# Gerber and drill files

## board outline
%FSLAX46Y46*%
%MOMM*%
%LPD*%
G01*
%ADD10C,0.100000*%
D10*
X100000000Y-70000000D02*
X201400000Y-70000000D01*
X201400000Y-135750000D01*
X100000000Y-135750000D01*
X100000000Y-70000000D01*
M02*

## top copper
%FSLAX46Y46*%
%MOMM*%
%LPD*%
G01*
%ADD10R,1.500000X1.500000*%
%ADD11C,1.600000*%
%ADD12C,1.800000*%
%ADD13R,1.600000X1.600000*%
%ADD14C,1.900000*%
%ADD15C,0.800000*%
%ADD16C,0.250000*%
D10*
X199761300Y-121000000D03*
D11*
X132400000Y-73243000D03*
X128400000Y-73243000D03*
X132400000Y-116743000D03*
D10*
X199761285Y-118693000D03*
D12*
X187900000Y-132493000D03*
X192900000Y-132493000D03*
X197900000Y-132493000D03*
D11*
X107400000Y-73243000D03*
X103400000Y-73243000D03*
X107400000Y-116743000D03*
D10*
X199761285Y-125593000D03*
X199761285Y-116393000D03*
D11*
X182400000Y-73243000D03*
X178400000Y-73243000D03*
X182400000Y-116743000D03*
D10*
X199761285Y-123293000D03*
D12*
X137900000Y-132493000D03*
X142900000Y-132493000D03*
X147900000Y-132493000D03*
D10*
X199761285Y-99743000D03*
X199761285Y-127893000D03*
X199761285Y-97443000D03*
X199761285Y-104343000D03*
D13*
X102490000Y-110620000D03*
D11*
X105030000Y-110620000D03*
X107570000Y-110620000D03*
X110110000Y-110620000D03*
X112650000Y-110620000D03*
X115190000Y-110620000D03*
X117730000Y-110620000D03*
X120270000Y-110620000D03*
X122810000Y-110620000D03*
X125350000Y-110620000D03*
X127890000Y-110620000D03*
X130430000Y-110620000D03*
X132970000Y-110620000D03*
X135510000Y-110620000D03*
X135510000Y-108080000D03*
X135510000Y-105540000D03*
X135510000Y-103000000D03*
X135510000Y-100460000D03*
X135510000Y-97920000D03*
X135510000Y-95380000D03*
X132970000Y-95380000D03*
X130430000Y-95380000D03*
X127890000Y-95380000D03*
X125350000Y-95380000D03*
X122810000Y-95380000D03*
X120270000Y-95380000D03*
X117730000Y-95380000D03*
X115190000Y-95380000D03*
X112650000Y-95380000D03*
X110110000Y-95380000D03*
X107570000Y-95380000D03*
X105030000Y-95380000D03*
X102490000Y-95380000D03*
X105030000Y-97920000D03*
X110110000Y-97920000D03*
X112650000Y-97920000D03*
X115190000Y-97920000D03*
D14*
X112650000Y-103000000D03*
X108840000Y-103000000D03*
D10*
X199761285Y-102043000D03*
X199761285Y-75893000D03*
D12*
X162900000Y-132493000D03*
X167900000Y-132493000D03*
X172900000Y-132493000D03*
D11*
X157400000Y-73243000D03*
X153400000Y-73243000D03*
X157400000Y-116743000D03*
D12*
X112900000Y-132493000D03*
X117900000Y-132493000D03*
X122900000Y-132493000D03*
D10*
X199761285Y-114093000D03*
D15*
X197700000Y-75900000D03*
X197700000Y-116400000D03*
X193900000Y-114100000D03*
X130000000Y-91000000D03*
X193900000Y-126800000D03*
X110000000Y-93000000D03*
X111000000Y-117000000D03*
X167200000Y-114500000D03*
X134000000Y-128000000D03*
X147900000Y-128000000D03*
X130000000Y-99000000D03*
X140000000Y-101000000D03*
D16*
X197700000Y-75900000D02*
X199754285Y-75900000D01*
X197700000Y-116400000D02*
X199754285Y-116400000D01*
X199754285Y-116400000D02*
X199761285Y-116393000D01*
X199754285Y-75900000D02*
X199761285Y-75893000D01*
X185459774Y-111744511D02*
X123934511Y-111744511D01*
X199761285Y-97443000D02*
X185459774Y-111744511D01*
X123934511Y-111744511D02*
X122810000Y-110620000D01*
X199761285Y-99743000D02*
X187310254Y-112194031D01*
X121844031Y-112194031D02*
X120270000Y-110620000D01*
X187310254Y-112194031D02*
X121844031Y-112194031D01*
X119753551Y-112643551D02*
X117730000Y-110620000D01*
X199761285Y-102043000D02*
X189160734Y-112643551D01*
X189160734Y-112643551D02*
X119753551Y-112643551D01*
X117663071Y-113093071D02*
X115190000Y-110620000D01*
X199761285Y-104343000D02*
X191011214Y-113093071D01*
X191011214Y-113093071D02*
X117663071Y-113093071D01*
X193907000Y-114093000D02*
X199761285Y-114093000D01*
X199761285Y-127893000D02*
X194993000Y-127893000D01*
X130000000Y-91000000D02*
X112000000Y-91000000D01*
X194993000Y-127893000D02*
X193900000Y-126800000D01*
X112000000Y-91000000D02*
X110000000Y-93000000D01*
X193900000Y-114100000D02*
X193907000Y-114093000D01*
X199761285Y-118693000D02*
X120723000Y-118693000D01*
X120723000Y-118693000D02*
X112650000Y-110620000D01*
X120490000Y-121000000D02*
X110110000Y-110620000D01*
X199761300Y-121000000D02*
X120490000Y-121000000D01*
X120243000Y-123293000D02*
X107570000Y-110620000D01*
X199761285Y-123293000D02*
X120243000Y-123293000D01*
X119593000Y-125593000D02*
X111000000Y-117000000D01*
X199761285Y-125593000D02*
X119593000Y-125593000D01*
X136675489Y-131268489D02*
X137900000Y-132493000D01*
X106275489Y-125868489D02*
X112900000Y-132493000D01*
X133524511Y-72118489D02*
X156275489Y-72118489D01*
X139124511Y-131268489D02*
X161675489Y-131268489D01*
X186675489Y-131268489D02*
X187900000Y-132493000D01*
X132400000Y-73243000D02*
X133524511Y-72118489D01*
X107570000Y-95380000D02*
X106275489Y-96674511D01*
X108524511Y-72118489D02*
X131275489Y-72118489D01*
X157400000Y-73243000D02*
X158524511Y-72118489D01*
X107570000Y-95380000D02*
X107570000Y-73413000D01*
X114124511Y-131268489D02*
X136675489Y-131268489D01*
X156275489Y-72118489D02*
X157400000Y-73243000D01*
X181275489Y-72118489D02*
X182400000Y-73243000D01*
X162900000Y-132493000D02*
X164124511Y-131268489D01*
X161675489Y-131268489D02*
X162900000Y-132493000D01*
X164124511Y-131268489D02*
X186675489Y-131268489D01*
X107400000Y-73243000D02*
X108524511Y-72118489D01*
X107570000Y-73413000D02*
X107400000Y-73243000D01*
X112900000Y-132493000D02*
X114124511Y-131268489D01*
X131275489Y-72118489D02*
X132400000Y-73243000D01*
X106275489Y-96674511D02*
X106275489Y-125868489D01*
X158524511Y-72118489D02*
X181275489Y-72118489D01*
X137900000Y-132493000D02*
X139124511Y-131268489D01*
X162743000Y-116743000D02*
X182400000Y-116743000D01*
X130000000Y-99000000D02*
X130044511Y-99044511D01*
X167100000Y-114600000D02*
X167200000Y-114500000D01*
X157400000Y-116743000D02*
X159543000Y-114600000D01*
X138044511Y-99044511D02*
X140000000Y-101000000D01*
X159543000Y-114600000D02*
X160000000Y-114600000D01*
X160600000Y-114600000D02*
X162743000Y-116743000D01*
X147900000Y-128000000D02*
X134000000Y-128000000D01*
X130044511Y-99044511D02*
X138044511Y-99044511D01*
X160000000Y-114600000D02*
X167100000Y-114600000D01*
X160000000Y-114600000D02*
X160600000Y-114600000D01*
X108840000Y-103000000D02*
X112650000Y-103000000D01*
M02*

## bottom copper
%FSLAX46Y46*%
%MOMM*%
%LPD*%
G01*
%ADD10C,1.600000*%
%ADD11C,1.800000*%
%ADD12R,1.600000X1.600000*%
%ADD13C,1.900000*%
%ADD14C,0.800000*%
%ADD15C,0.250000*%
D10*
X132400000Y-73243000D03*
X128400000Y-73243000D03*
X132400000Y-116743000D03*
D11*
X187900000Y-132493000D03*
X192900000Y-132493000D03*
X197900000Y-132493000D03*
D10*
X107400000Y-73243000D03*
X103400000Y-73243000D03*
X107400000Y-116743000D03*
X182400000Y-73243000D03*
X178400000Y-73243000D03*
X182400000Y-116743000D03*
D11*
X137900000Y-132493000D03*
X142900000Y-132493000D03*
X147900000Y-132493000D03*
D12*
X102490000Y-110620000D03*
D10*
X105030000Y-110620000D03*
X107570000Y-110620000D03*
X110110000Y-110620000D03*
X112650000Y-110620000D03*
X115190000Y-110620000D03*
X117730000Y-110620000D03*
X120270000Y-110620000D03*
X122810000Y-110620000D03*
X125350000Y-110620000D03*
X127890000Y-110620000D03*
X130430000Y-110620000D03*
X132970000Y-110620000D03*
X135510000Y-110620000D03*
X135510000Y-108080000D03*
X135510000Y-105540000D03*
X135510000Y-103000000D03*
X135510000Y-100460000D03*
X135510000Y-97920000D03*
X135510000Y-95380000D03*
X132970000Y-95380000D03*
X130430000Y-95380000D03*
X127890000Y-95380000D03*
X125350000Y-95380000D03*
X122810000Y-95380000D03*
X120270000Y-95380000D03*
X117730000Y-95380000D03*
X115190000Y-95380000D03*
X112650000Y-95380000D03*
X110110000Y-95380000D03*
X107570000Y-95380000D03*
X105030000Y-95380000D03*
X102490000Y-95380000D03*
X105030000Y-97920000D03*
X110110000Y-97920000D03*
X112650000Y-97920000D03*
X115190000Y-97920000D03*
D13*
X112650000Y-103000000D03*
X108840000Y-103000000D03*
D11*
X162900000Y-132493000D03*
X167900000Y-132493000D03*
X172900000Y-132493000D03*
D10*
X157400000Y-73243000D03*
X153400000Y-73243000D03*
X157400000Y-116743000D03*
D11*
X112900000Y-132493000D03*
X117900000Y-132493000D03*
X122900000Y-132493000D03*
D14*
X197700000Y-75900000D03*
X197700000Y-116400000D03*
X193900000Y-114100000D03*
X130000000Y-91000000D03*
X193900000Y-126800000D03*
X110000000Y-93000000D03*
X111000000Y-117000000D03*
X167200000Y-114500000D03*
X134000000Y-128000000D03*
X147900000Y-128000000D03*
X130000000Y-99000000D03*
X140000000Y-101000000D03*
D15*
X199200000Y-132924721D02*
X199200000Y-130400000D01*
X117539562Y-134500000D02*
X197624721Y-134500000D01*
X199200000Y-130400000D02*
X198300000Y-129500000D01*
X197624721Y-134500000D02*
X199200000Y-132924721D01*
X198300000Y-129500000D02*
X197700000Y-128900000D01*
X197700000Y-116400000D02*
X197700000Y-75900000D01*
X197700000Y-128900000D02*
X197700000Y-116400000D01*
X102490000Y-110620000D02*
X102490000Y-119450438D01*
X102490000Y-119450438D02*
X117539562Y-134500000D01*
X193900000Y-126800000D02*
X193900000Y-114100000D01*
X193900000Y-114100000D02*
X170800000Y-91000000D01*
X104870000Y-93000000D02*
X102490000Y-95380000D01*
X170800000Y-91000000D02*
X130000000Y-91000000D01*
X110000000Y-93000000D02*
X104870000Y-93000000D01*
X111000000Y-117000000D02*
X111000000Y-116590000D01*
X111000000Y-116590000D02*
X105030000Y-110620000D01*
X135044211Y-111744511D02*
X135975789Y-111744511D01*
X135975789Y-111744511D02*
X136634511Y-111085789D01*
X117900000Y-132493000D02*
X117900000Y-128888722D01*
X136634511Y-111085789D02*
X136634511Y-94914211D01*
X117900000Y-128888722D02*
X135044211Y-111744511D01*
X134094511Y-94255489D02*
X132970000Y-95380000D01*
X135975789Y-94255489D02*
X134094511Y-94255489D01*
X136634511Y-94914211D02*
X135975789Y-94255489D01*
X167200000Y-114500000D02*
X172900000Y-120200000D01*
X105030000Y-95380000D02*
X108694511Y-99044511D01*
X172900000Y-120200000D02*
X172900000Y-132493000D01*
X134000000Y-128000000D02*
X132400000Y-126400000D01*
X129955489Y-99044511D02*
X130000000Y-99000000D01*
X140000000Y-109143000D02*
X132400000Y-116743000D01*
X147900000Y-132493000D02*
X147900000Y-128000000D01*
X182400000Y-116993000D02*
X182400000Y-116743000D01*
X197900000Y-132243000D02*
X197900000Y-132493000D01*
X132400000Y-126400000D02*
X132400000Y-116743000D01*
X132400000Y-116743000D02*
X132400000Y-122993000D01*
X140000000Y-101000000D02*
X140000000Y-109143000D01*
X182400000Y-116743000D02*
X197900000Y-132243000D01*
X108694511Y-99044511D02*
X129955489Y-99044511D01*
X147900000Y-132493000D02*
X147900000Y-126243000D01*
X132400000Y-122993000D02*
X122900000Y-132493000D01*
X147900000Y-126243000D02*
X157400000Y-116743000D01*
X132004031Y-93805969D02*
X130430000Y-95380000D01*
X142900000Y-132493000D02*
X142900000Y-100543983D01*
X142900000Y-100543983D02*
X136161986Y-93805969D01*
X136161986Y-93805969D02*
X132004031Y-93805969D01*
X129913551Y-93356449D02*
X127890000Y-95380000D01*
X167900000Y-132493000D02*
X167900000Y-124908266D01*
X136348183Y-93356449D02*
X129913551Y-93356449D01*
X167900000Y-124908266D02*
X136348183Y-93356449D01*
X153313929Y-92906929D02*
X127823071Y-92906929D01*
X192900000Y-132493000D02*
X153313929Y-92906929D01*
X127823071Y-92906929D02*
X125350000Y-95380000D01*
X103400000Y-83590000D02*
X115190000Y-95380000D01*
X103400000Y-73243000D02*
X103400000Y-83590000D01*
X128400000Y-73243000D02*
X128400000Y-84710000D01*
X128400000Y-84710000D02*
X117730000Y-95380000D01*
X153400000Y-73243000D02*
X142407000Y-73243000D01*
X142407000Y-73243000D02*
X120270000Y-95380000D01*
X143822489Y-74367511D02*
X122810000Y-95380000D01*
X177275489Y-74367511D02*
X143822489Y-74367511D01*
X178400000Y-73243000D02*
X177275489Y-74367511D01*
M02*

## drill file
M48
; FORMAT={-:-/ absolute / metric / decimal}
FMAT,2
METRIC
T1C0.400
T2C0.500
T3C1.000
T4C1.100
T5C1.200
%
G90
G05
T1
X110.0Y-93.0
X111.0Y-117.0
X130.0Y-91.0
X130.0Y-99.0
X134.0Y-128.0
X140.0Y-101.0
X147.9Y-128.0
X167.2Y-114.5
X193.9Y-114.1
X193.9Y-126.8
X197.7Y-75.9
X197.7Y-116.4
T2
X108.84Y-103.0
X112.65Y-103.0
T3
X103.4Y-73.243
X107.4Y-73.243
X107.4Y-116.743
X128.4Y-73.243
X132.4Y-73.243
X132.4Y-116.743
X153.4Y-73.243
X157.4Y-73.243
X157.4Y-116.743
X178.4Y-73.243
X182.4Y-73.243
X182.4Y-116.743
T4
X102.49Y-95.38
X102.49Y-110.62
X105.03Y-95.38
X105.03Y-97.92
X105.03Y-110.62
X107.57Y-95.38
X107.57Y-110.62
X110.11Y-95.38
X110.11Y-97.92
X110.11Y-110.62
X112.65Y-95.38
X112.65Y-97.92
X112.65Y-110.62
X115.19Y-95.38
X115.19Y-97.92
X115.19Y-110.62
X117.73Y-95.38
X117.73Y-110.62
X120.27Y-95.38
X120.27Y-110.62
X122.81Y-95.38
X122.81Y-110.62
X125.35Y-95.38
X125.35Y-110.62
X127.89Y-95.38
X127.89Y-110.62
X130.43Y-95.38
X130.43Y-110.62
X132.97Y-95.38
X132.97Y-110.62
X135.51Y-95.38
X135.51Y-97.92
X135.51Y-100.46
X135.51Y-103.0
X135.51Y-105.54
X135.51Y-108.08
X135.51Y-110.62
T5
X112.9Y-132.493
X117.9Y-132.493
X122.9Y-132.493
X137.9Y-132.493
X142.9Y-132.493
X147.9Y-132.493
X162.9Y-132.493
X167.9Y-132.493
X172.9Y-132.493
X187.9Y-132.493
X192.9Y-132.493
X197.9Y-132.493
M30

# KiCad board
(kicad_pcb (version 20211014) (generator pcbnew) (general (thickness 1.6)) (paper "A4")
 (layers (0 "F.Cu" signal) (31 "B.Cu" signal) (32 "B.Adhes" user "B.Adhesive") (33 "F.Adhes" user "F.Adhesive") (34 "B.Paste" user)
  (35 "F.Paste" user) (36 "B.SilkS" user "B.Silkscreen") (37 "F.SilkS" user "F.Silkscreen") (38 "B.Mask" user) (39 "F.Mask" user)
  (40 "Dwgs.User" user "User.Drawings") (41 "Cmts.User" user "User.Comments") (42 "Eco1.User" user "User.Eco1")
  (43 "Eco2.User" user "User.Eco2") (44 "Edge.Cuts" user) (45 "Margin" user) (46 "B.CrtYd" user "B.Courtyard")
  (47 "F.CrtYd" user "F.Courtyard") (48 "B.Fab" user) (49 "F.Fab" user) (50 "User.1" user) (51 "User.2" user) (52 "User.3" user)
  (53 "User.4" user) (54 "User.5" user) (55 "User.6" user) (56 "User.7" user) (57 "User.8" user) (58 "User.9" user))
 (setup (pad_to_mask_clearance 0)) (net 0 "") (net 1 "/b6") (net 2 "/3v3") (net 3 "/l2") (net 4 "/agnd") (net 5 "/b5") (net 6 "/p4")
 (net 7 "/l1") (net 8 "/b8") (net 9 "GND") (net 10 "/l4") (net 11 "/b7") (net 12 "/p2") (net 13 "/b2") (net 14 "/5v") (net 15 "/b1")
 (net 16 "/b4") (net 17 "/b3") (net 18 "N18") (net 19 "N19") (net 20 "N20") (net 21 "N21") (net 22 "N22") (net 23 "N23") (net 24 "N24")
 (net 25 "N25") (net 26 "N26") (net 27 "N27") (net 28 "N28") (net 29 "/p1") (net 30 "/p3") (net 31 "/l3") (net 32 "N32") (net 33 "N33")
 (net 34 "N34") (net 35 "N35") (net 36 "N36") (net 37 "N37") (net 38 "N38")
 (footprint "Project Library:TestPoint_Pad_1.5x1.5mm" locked (layer "F.Cu") (at 199.7613 121)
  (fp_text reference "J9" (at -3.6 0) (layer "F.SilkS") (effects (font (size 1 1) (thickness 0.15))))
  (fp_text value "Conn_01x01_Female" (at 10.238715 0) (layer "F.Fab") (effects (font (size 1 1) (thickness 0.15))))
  (pad "1" smd rect locked (at 0 0) (size 1.5 1.5) (layers "F.Cu" "F.Mask") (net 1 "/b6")))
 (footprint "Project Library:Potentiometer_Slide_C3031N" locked (layer "F.Cu") (at 132.4 73.243)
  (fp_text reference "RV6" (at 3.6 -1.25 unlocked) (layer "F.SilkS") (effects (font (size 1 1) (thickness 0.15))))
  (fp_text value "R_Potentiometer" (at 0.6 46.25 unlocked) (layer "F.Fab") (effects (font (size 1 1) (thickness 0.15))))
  (pad "1" thru_hole circle locked (at 0 0) (size 1.6 1.6) (drill 1) (layers *.Cu *.Mask) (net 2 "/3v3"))
  (pad "2" thru_hole circle locked (at -4 0) (size 1.6 1.6) (drill 1) (layers *.Cu *.Mask) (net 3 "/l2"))
  (pad "3" thru_hole circle locked (at 0 43.5) (size 1.6 1.6) (drill 1) (layers *.Cu *.Mask) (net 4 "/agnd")))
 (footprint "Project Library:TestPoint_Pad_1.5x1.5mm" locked (layer "F.Cu") (at 199.761285 118.693)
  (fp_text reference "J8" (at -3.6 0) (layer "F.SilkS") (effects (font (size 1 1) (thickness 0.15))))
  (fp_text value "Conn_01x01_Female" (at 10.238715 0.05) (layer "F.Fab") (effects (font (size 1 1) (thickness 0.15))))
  (pad "1" smd rect locked (at 0 0) (size 1.5 1.5) (layers "F.Cu" "F.Mask") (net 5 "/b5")))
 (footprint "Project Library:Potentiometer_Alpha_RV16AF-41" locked (layer "F.Cu") (at 187.9 132.493)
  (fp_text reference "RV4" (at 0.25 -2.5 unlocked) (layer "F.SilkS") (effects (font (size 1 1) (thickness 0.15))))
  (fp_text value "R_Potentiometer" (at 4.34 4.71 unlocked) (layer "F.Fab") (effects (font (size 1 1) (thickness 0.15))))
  (pad "1" thru_hole circle locked (at 0 0) (size 1.8 1.8) (drill 1.2) (layers *.Cu *.Mask) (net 2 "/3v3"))
  (pad "2" thru_hole circle locked (at 5 0) (size 1.8 1.8) (drill 1.2) (layers *.Cu *.Mask) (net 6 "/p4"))
  (pad "3" thru_hole circle locked (at 10 0) (size 1.8 1.8) (drill 1.2) (layers *.Cu *.Mask) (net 4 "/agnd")))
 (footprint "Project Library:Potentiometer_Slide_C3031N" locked (layer "F.Cu") (at 107.4 73.243)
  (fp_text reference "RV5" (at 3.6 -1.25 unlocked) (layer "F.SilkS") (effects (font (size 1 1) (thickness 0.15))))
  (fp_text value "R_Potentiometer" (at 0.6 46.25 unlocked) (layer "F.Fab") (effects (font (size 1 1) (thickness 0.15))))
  (pad "1" thru_hole circle locked (at 0 0) (size 1.6 1.6) (drill 1) (layers *.Cu *.Mask) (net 2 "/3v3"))
  (pad "2" thru_hole circle locked (at -4 0) (size 1.6 1.6) (drill 1) (layers *.Cu *.Mask) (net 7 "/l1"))
  (pad "3" thru_hole circle locked (at 0 43.5) (size 1.6 1.6) (drill 1) (layers *.Cu *.Mask) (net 4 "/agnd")))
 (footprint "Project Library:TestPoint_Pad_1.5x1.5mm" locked (layer "F.Cu") (at 199.761285 125.593)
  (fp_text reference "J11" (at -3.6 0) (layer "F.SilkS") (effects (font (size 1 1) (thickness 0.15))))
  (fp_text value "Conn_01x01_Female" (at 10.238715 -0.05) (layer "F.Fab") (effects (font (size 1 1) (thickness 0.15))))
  (pad "1" smd rect locked (at 0 0) (size 1.5 1.5) (layers "F.Cu" "F.Mask") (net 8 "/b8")))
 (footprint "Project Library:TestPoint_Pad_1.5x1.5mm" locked (layer "F.Cu") (at 199.761285 116.393)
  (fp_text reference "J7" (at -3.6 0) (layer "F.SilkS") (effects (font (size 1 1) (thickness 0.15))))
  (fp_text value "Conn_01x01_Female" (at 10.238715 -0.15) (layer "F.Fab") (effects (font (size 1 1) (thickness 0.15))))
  (pad "1" smd rect locked (at 0 0) (size 1.5 1.5) (layers "F.Cu" "F.Mask") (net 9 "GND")))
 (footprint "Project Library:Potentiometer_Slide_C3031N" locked (layer "F.Cu") (at 182.4 73.243)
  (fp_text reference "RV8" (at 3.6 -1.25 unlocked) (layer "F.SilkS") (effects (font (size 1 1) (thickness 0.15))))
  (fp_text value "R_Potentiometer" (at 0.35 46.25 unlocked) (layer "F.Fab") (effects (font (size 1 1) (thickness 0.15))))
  (pad "1" thru_hole circle locked (at 0 0) (size 1.6 1.6) (drill 1) (layers *.Cu *.Mask) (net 2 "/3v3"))
  (pad "2" thru_hole circle locked (at -4 0) (size 1.6 1.6) (drill 1) (layers *.Cu *.Mask) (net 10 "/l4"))
  (pad "3" thru_hole circle locked (at 0 43.5) (size 1.6 1.6) (drill 1) (layers *.Cu *.Mask) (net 4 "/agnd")))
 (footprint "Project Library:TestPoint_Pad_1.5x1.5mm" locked (layer "F.Cu") (at 199.761285 123.293)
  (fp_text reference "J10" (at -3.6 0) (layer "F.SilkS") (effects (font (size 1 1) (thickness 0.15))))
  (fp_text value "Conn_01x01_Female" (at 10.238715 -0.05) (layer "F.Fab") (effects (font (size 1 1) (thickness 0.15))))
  (pad "1" smd rect locked (at 0 0) (size 1.5 1.5) (layers "F.Cu" "F.Mask") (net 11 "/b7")))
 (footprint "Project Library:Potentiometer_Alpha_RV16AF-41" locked (layer "F.Cu") (at 137.9 132.493)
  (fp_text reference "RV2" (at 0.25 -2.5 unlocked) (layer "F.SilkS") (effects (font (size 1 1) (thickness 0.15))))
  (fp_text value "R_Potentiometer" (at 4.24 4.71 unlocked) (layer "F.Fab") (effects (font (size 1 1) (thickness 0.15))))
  (pad "1" thru_hole circle locked (at 0 0) (size 1.8 1.8) (drill 1.2) (layers *.Cu *.Mask) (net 2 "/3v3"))
  (pad "2" thru_hole circle locked (at 5 0) (size 1.8 1.8) (drill 1.2) (layers *.Cu *.Mask) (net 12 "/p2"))
  (pad "3" thru_hole circle locked (at 10 0) (size 1.8 1.8) (drill 1.2) (layers *.Cu *.Mask) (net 4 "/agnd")))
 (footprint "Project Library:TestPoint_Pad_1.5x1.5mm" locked (layer "F.Cu") (at 199.761285 99.743)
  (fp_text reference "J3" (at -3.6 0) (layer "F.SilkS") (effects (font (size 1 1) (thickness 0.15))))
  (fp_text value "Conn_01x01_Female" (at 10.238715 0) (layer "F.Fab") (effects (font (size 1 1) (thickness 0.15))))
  (pad "1" smd rect locked (at 0 0) (size 1.5 1.5) (layers "F.Cu" "F.Mask") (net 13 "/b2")))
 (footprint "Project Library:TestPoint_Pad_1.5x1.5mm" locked (layer "F.Cu") (at 199.761285 127.893)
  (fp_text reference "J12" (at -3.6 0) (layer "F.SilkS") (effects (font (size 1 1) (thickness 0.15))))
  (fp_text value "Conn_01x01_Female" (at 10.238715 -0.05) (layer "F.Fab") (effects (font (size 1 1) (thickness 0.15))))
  (pad "1" smd rect locked (at 0 0) (size 1.5 1.5) (layers "F.Cu" "F.Mask") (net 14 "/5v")))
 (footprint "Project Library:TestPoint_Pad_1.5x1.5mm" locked (layer "F.Cu") (at 199.761285 97.443)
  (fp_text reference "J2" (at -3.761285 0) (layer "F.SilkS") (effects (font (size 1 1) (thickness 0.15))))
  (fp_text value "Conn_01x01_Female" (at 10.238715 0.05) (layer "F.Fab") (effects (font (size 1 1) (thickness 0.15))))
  (pad "1" smd rect locked (at 0 0) (size 1.5 1.5) (layers "F.Cu" "F.Mask") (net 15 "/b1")))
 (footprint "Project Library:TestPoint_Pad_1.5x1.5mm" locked (layer "F.Cu") (at 199.761285 104.343)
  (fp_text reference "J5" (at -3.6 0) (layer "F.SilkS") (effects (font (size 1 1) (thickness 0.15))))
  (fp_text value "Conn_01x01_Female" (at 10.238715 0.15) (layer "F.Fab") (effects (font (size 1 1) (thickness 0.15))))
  (pad "1" smd rect locked (at 0 0) (size 1.5 1.5) (layers "F.Cu" "F.Mask") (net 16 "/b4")))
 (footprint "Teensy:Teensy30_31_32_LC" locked (layer "F.Cu") (at 119 103)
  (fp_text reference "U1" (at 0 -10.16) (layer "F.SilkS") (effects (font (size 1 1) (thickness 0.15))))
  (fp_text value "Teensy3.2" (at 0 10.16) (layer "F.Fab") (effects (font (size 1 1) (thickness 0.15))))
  (pad "1" thru_hole rect locked (at -16.51 7.62) (size 1.6 1.6) (drill 1.1) (layers *.Cu *.Mask) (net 9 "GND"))
  (pad "2" thru_hole circle locked (at -13.97 7.62) (size 1.6 1.6) (drill 1.1) (layers *.Cu *.Mask) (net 8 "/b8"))
  (pad "3" thru_hole circle locked (at -11.43 7.62) (size 1.6 1.6) (drill 1.1) (layers *.Cu *.Mask) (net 11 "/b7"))
  (pad "4" thru_hole circle locked (at -8.89 7.62) (size 1.6 1.6) (drill 1.1) (layers *.Cu *.Mask) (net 1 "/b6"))
  (pad "5" thru_hole circle locked (at -6.35 7.62) (size 1.6 1.6) (drill 1.1) (layers *.Cu *.Mask) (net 5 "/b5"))
  (pad "6" thru_hole circle locked (at -3.81 7.62) (size 1.6 1.6) (drill 1.1) (layers *.Cu *.Mask) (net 16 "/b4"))
  (pad "7" thru_hole circle locked (at -1.27 7.62) (size 1.6 1.6) (drill 1.1) (layers *.Cu *.Mask) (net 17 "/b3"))
  (pad "8" thru_hole circle locked (at 1.27 7.62) (size 1.6 1.6) (drill 1.1) (layers *.Cu *.Mask) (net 13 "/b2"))
  (pad "9" thru_hole circle locked (at 3.81 7.62) (size 1.6 1.6) (drill 1.1) (layers *.Cu *.Mask) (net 15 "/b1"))
  (pad "10" thru_hole circle locked (at 6.35 7.62) (size 1.6 1.6) (drill 1.1) (layers *.Cu *.Mask) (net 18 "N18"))
  (pad "11" thru_hole circle locked (at 8.89 7.62) (size 1.6 1.6) (drill 1.1) (layers *.Cu *.Mask) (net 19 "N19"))
  (pad "12" thru_hole circle locked (at 11.43 7.62) (size 1.6 1.6) (drill 1.1) (layers *.Cu *.Mask) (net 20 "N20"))
  (pad "13" thru_hole circle locked (at 13.97 7.62) (size 1.6 1.6) (drill 1.1) (layers *.Cu *.Mask) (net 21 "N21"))
  (pad "14" thru_hole circle locked (at 16.51 7.62) (size 1.6 1.6) (drill 1.1) (layers *.Cu *.Mask) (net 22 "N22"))
  (pad "15" thru_hole circle locked (at 16.51 5.08) (size 1.6 1.6) (drill 1.1) (layers *.Cu *.Mask) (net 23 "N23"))
  (pad "16" thru_hole circle locked (at 16.51 2.54) (size 1.6 1.6) (drill 1.1) (layers *.Cu *.Mask) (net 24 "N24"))
  (pad "17" thru_hole circle locked (at 16.51 0) (size 1.6 1.6) (drill 1.1) (layers *.Cu *.Mask) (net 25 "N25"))
  (pad "18" thru_hole circle locked (at 16.51 -2.54) (size 1.6 1.6) (drill 1.1) (layers *.Cu *.Mask) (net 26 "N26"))
  (pad "19" thru_hole circle locked (at 16.51 -5.08) (size 1.6 1.6) (drill 1.1) (layers *.Cu *.Mask) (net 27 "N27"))
  (pad "20" thru_hole circle locked (at 16.51 -7.62) (size 1.6 1.6) (drill 1.1) (layers *.Cu *.Mask) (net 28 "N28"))
  (pad "21" thru_hole circle locked (at 13.97 -7.62) (size 1.6 1.6) (drill 1.1) (layers *.Cu *.Mask) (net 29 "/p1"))
  (pad "22" thru_hole circle locked (at 11.43 -7.62) (size 1.6 1.6) (drill 1.1) (layers *.Cu *.Mask) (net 12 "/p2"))
  (pad "23" thru_hole circle locked (at 8.89 -7.62) (size 1.6 1.6) (drill 1.1) (layers *.Cu *.Mask) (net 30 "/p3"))
  (pad "24" thru_hole circle locked (at 6.35 -7.62) (size 1.6 1.6) (drill 1.1) (layers *.Cu *.Mask) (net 6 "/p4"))
  (pad "25" thru_hole circle locked (at 3.81 -7.62) (size 1.6 1.6) (drill 1.1) (layers *.Cu *.Mask) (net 10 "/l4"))
  (pad "26" thru_hole circle locked (at 1.27 -7.62) (size 1.6 1.6) (drill 1.1) (layers *.Cu *.Mask) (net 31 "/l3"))
  (pad "27" thru_hole circle locked (at -1.27 -7.62) (size 1.6 1.6) (drill 1.1) (layers *.Cu *.Mask) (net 3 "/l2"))
  (pad "28" thru_hole circle locked (at -3.81 -7.62) (size 1.6 1.6) (drill 1.1) (layers *.Cu *.Mask) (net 7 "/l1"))
  (pad "29" thru_hole circle locked (at -6.35 -7.62) (size 1.6 1.6) (drill 1.1) (layers *.Cu *.Mask) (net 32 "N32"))
  (pad "30" thru_hole circle locked (at -8.89 -7.62) (size 1.6 1.6) (drill 1.1) (layers *.Cu *.Mask) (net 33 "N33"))
  (pad "31" thru_hole circle locked (at -11.43 -7.62) (size 1.6 1.6) (drill 1.1) (layers *.Cu *.Mask) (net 2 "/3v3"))
  (pad "32" thru_hole circle locked (at -13.97 -7.62) (size 1.6 1.6) (drill 1.1) (layers *.Cu *.Mask) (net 4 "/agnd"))
  (pad "33" thru_hole circle locked (at -16.51 -7.62) (size 1.6 1.6) (drill 1.1) (layers *.Cu *.Mask) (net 14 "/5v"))
  (pad "34" thru_hole circle locked (at -13.97 -5.08) (size 1.6 1.6) (drill 1.1) (layers *.Cu *.Mask) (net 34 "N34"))
  (pad "35" thru_hole circle locked (at -8.89 -5.08) (size 1.6 1.6) (drill 1.1) (layers *.Cu *.Mask) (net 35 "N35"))
  (pad "36" thru_hole circle locked (at -6.35 -5.08) (size 1.6 1.6) (drill 1.1) (layers *.Cu *.Mask) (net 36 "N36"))
  (pad "37" thru_hole circle locked (at -3.81 -5.08) (size 1.6 1.6) (drill 1.1) (layers *.Cu *.Mask) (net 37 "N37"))
  (pad "38" thru_hole circle locked (at -6.35 0) (size 1.9 1.9) (drill 0.5) (layers *.Cu *.Mask) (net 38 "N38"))
  (pad "38" thru_hole circle locked (at -10.16 0) (size 1.9 1.9) (drill 0.5) (layers *.Cu *.Mask) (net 38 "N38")))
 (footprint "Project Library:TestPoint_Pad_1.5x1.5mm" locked (layer "F.Cu") (at 199.761285 102.043)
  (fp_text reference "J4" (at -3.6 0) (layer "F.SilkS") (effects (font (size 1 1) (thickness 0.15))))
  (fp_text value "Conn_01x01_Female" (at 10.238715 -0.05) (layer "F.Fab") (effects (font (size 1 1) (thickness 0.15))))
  (pad "1" smd rect locked (at 0 0) (size 1.5 1.5) (layers "F.Cu" "F.Mask") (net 17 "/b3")))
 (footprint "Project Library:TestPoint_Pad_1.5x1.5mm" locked (layer "F.Cu") (at 199.761285 75.893)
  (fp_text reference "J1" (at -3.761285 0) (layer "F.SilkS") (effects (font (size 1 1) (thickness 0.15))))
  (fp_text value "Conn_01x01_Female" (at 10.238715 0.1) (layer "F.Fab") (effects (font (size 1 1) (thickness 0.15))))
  (pad "1" smd rect locked (at 0 0) (size 1.5 1.5) (layers "F.Cu" "F.Mask") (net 9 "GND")))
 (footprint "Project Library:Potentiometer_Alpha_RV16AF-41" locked (layer "F.Cu") (at 162.9 132.493)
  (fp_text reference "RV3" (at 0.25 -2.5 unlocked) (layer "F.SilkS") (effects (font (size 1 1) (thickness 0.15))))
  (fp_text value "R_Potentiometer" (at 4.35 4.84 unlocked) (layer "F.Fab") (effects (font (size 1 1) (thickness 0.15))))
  (pad "1" thru_hole circle locked (at 0 0) (size 1.8 1.8) (drill 1.2) (layers *.Cu *.Mask) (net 2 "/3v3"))
  (pad "2" thru_hole circle locked (at 5 0) (size 1.8 1.8) (drill 1.2) (layers *.Cu *.Mask) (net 30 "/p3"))
  (pad "3" thru_hole circle locked (at 10 0) (size 1.8 1.8) (drill 1.2) (layers *.Cu *.Mask) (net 4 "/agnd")))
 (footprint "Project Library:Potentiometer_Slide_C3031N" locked (layer "F.Cu") (at 157.4 73.243)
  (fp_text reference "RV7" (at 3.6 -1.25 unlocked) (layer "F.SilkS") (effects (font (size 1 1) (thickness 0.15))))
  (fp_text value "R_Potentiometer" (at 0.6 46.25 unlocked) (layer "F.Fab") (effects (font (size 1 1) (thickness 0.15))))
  (pad "1" thru_hole circle locked (at 0 0) (size 1.6 1.6) (drill 1) (layers *.Cu *.Mask) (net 2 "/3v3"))
  (pad "2" thru_hole circle locked (at -4 0) (size 1.6 1.6) (drill 1) (layers *.Cu *.Mask) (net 31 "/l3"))
  (pad "3" thru_hole circle locked (at 0 43.5) (size 1.6 1.6) (drill 1) (layers *.Cu *.Mask) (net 4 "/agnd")))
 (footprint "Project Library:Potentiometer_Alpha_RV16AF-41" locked (layer "F.Cu") (at 112.9 132.493)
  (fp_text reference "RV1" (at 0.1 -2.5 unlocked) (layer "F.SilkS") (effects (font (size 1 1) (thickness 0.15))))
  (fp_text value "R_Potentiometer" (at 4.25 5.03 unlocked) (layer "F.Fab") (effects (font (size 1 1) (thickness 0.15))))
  (pad "1" thru_hole circle locked (at 0 0) (size 1.8 1.8) (drill 1.2) (layers *.Cu *.Mask) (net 2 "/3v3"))
  (pad "2" thru_hole circle locked (at 5 0) (size 1.8 1.8) (drill 1.2) (layers *.Cu *.Mask) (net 29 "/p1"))
  (pad "3" thru_hole circle locked (at 10 0) (size 1.8 1.8) (drill 1.2) (layers *.Cu *.Mask) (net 4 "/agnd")))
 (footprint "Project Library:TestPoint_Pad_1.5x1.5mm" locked (layer "F.Cu") (at 199.761285 114.093)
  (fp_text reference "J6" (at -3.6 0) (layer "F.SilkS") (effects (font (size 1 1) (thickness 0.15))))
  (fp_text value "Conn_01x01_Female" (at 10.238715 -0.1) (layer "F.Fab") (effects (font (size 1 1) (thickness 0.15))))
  (pad "1" smd rect locked (at 0 0) (size 1.5 1.5) (layers "F.Cu" "F.Mask") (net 14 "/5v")))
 (gr_rect locked (start 100 70) (end 201.4 135.75) (layer "Edge.Cuts") (width 0.1) (fill none))
 (segment (start 197.7 75.9) (end 199.754285 75.9) (width 0.25) (layer "F.Cu") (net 9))
 (segment (start 197.7 116.4) (end 199.754285 116.4) (width 0.25) (layer "F.Cu") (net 9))
 (segment (start 199.754285 116.4) (end 199.761285 116.393) (width 0.25) (layer "F.Cu") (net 9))
 (segment (start 199.754285 75.9) (end 199.761285 75.893) (width 0.25) (layer "F.Cu") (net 9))
 (via (at 197.7 75.9) (size 0.8) (drill 0.4) (layers "F.Cu" "B.Cu") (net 9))
 (via (at 197.7 116.4) (size 0.8) (drill 0.4) (layers "F.Cu" "B.Cu") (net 9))
 (segment (start 199.2 132.924721) (end 199.2 130.4) (width 0.25) (layer "B.Cu") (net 9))
 (segment (start 117.539562 134.5) (end 197.624721 134.5) (width 0.25) (layer "B.Cu") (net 9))
 (segment (start 199.2 130.4) (end 198.3 129.5) (width 0.25) (layer "B.Cu") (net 9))
 (segment (start 197.624721 134.5) (end 199.2 132.924721) (width 0.25) (layer "B.Cu") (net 9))
 (segment (start 198.3 129.5) (end 197.7 128.9) (width 0.25) (layer "B.Cu") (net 9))
 (segment (start 197.7 116.4) (end 197.7 75.9) (width 0.25) (layer "B.Cu") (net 9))
 (segment (start 197.7 128.9) (end 197.7 116.4) (width 0.25) (layer "B.Cu") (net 9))
 (segment (start 102.49 110.62) (end 102.49 119.450438) (width 0.25) (layer "B.Cu") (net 9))
 (segment (start 102.49 119.450438) (end 117.539562 134.5) (width 0.25) (layer "B.Cu") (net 9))
 (segment (start 185.459774 111.744511) (end 123.934511 111.744511) (width 0.25) (layer "F.Cu") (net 15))
 (segment (start 199.761285 97.443) (end 185.459774 111.744511) (width 0.25) (layer "F.Cu") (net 15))
 (segment (start 123.934511 111.744511) (end 122.81 110.62) (width 0.25) (layer "F.Cu") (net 15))
 (segment (start 199.761285 99.743) (end 187.310254 112.194031) (width 0.25) (layer "F.Cu") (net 13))
 (segment (start 121.844031 112.194031) (end 120.27 110.62) (width 0.25) (layer "F.Cu") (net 13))
 (segment (start 187.310254 112.194031) (end 121.844031 112.194031) (width 0.25) (layer "F.Cu") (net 13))
 (segment (start 119.753551 112.643551) (end 117.73 110.62) (width 0.25) (layer "F.Cu") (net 17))
 (segment (start 199.761285 102.043) (end 189.160734 112.643551) (width 0.25) (layer "F.Cu") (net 17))
 (segment (start 189.160734 112.643551) (end 119.753551 112.643551) (width 0.25) (layer "F.Cu") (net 17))
 (segment (start 117.663071 113.093071) (end 115.19 110.62) (width 0.25) (layer "F.Cu") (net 16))
 (segment (start 199.761285 104.343) (end 191.011214 113.093071) (width 0.25) (layer "F.Cu") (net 16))
 (segment (start 191.011214 113.093071) (end 117.663071 113.093071) (width 0.25) (layer "F.Cu") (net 16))
 (segment (start 193.907 114.093) (end 199.761285 114.093) (width 0.25) (layer "F.Cu") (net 14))
 (segment (start 199.761285 127.893) (end 194.993 127.893) (width 0.25) (layer "F.Cu") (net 14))
 (segment (start 130 91) (end 112 91) (width 0.25) (layer "F.Cu") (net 14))
 (segment (start 194.993 127.893) (end 193.9 126.8) (width 0.25) (layer "F.Cu") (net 14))
 (segment (start 112 91) (end 110 93) (width 0.25) (layer "F.Cu") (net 14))
 (segment (start 193.9 114.1) (end 193.907 114.093) (width 0.25) (layer "F.Cu") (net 14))
 (via (at 193.9 114.1) (size 0.8) (drill 0.4) (layers "F.Cu" "B.Cu") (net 14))
 (via (at 130 91) (size 0.8) (drill 0.4) (layers "F.Cu" "B.Cu") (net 14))
 (via (at 193.9 126.8) (size 0.8) (drill 0.4) (layers "F.Cu" "B.Cu") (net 14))
 (via (at 110 93) (size 0.8) (drill 0.4) (layers "F.Cu" "B.Cu") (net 14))
 (segment (start 193.9 126.8) (end 193.9 114.1) (width 0.25) (layer "B.Cu") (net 14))
 (segment (start 193.9 114.1) (end 170.8 91) (width 0.25) (layer "B.Cu") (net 14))
 (segment (start 104.87 93) (end 102.49 95.38) (width 0.25) (layer "B.Cu") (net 14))
 (segment (start 170.8 91) (end 130 91) (width 0.25) (layer "B.Cu") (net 14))
 (segment (start 110 93) (end 104.87 93) (width 0.25) (layer "B.Cu") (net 14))
 (segment (start 199.761285 118.693) (end 120.723 118.693) (width 0.25) (layer "F.Cu") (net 5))
 (segment (start 120.723 118.693) (end 112.65 110.62) (width 0.25) (layer "F.Cu") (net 5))
 (segment (start 120.49 121) (end 110.11 110.62) (width 0.25) (layer "F.Cu") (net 1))
 (segment (start 199.7613 121) (end 120.49 121) (width 0.25) (layer "F.Cu") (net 1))
 (segment (start 120.243 123.293) (end 107.57 110.62) (width 0.25) (layer "F.Cu") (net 11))
 (segment (start 199.761285 123.293) (end 120.243 123.293) (width 0.25) (layer "F.Cu") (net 11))
 (segment (start 119.593 125.593) (end 111 117) (width 0.25) (layer "F.Cu") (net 8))
 (segment (start 199.761285 125.593) (end 119.593 125.593) (width 0.25) (layer "F.Cu") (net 8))
 (via (at 111 117) (size 0.8) (drill 0.4) (layers "F.Cu" "B.Cu") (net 8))
 (segment (start 111 117) (end 111 116.59) (width 0.25) (layer "B.Cu") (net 8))
 (segment (start 111 116.59) (end 105.03 110.62) (width 0.25) (layer "B.Cu") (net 8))
 (segment (start 136.675489 131.268489) (end 137.9 132.493) (width 0.25) (layer "F.Cu") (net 2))
 (segment (start 106.275489 125.868489) (end 112.9 132.493) (width 0.25) (layer "F.Cu") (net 2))
 (segment (start 133.524511 72.118489) (end 156.275489 72.118489) (width 0.25) (layer "F.Cu") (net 2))
 (segment (start 139.124511 131.268489) (end 161.675489 131.268489) (width 0.25) (layer "F.Cu") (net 2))
 (segment (start 186.675489 131.268489) (end 187.9 132.493) (width 0.25) (layer "F.Cu") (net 2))
 (segment (start 132.4 73.243) (end 133.524511 72.118489) (width 0.25) (layer "F.Cu") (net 2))
 (segment (start 107.57 95.38) (end 106.275489 96.674511) (width 0.25) (layer "F.Cu") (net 2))
 (segment (start 108.524511 72.118489) (end 131.275489 72.118489) (width 0.25) (layer "F.Cu") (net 2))
 (segment (start 157.4 73.243) (end 158.524511 72.118489) (width 0.25) (layer "F.Cu") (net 2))
 (segment (start 107.57 95.38) (end 107.57 73.413) (width 0.25) (layer "F.Cu") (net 2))
 (segment (start 114.124511 131.268489) (end 136.675489 131.268489) (width 0.25) (layer "F.Cu") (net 2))
 (segment (start 156.275489 72.118489) (end 157.4 73.243) (width 0.25) (layer "F.Cu") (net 2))
 (segment (start 181.275489 72.118489) (end 182.4 73.243) (width 0.25) (layer "F.Cu") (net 2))
 (segment (start 162.9 132.493) (end 164.124511 131.268489) (width 0.25) (layer "F.Cu") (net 2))
 (segment (start 161.675489 131.268489) (end 162.9 132.493) (width 0.25) (layer "F.Cu") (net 2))
 (segment (start 164.124511 131.268489) (end 186.675489 131.268489) (width 0.25) (layer "F.Cu") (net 2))
 (segment (start 107.4 73.243) (end 108.524511 72.118489) (width 0.25) (layer "F.Cu") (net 2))
 (segment (start 107.57 73.413) (end 107.4 73.243) (width 0.25) (layer "F.Cu") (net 2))
 (segment (start 112.9 132.493) (end 114.124511 131.268489) (width 0.25) (layer "F.Cu") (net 2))
 (segment (start 131.275489 72.118489) (end 132.4 73.243) (width 0.25) (layer "F.Cu") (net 2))
 (segment (start 106.275489 96.674511) (end 106.275489 125.868489) (width 0.25) (layer "F.Cu") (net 2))
 (segment (start 158.524511 72.118489) (end 181.275489 72.118489) (width 0.25) (layer "F.Cu") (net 2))
 (segment (start 137.9 132.493) (end 139.124511 131.268489) (width 0.25) (layer "F.Cu") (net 2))
 (segment (start 135.044211 111.744511) (end 135.975789 111.744511) (width 0.25) (layer "B.Cu") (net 29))
 (segment (start 135.975789 111.744511) (end 136.634511 111.085789) (width 0.25) (layer "B.Cu") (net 29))
 (segment (start 117.9 132.493) (end 117.9 128.888722) (width 0.25) (layer "B.Cu") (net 29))
 (segment (start 136.634511 111.085789) (end 136.634511 94.914211) (width 0.25) (layer "B.Cu") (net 29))
 (segment (start 117.9 128.888722) (end 135.044211 111.744511) (width 0.25) (layer "B.Cu") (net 29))
 (segment (start 134.094511 94.255489) (end 132.97 95.38) (width 0.25) (layer "B.Cu") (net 29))
 (segment (start 135.975789 94.255489) (end 134.094511 94.255489) (width 0.25) (layer "B.Cu") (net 29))
 (segment (start 136.634511 94.914211) (end 135.975789 94.255489) (width 0.25) (layer "B.Cu") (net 29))
 (segment (start 162.743 116.743) (end 182.4 116.743) (width 0.25) (layer "F.Cu") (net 4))
 (segment (start 130 99) (end 130.044511 99.044511) (width 0.25) (layer "F.Cu") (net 4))
 (segment (start 167.1 114.6) (end 167.2 114.5) (width 0.25) (layer "F.Cu") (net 4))
 (segment (start 157.4 116.743) (end 159.543 114.6) (width 0.25) (layer "F.Cu") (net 4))
 (segment (start 138.044511 99.044511) (end 140 101) (width 0.25) (layer "F.Cu") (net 4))
 (segment (start 159.543 114.6) (end 160 114.6) (width 0.25) (layer "F.Cu") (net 4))
 (segment (start 160.6 114.6) (end 162.743 116.743) (width 0.25) (layer "F.Cu") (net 4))
 (segment (start 147.9 128) (end 134 128) (width 0.25) (layer "F.Cu") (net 4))
 (segment (start 130.044511 99.044511) (end 138.044511 99.044511) (width 0.25) (layer "F.Cu") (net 4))
 (segment (start 160 114.6) (end 167.1 114.6) (width 0.25) (layer "F.Cu") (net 4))
 (segment (start 160 114.6) (end 160.6 114.6) (width 0.25) (layer "F.Cu") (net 4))
 (via (at 167.2 114.5) (size 0.8) (drill 0.4) (layers "F.Cu" "B.Cu") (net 4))
 (via (at 134 128) (size 0.8) (drill 0.4) (layers "F.Cu" "B.Cu") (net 4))
 (via (at 147.9 128) (size 0.8) (drill 0.4) (layers "F.Cu" "B.Cu") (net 4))
 (via (at 130 99) (size 0.8) (drill 0.4) (layers "F.Cu" "B.Cu") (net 4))
 (via (at 140 101) (size 0.8) (drill 0.4) (layers "F.Cu" "B.Cu") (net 4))
 (segment (start 167.2 114.5) (end 172.9 120.2) (width 0.25) (layer "B.Cu") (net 4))
 (segment (start 105.03 95.38) (end 108.694511 99.044511) (width 0.25) (layer "B.Cu") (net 4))
 (segment (start 172.9 120.2) (end 172.9 132.493) (width 0.25) (layer "B.Cu") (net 4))
 (segment (start 134 128) (end 132.4 126.4) (width 0.25) (layer "B.Cu") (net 4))
 (segment (start 129.955489 99.044511) (end 130 99) (width 0.25) (layer "B.Cu") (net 4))
 (segment (start 140 109.143) (end 132.4 116.743) (width 0.25) (layer "B.Cu") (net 4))
 (segment (start 147.9 132.493) (end 147.9 128) (width 0.25) (layer "B.Cu") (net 4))
 (segment (start 182.4 116.993) (end 182.4 116.743) (width 0.25) (layer "B.Cu") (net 4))
 (segment (start 197.9 132.243) (end 197.9 132.493) (width 0.25) (layer "B.Cu") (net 4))
 (segment (start 132.4 126.4) (end 132.4 116.743) (width 0.25) (layer "B.Cu") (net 4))
 (segment (start 132.4 116.743) (end 132.4 122.993) (width 0.25) (layer "B.Cu") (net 4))
 (segment (start 140 101) (end 140 109.143) (width 0.25) (layer "B.Cu") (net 4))
 (segment (start 182.4 116.743) (end 197.9 132.243) (width 0.25) (layer "B.Cu") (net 4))
 (segment (start 108.694511 99.044511) (end 129.955489 99.044511) (width 0.25) (layer "B.Cu") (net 4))
 (segment (start 147.9 132.493) (end 147.9 126.243) (width 0.25) (layer "B.Cu") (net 4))
 (segment (start 132.4 122.993) (end 122.9 132.493) (width 0.25) (layer "B.Cu") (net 4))
 (segment (start 147.9 126.243) (end 157.4 116.743) (width 0.25) (layer "B.Cu") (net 4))
 (segment (start 132.004031 93.805969) (end 130.43 95.38) (width 0.25) (layer "B.Cu") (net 12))
 (segment (start 142.9 132.493) (end 142.9 100.543983) (width 0.25) (layer "B.Cu") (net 12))
 (segment (start 142.9 100.543983) (end 136.161986 93.805969) (width 0.25) (layer "B.Cu") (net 12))
 (segment (start 136.161986 93.805969) (end 132.004031 93.805969) (width 0.25) (layer "B.Cu") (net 12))
 (segment (start 129.913551 93.356449) (end 127.89 95.38) (width 0.25) (layer "B.Cu") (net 30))
 (segment (start 167.9 132.493) (end 167.9 124.908266) (width 0.25) (layer "B.Cu") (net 30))
 (segment (start 136.348183 93.356449) (end 129.913551 93.356449) (width 0.25) (layer "B.Cu") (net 30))
 (segment (start 167.9 124.908266) (end 136.348183 93.356449) (width 0.25) (layer "B.Cu") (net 30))
 (segment (start 153.313929 92.906929) (end 127.823071 92.906929) (width 0.25) (layer "B.Cu") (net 6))
 (segment (start 192.9 132.493) (end 153.313929 92.906929) (width 0.25) (layer "B.Cu") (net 6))
 (segment (start 127.823071 92.906929) (end 125.35 95.38) (width 0.25) (layer "B.Cu") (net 6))
 (segment (start 103.4 83.59) (end 115.19 95.38) (width 0.25) (layer "B.Cu") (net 7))
 (segment (start 103.4 73.243) (end 103.4 83.59) (width 0.25) (layer "B.Cu") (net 7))
 (segment (start 128.4 73.243) (end 128.4 84.71) (width 0.25) (layer "B.Cu") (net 3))
 (segment (start 128.4 84.71) (end 117.73 95.38) (width 0.25) (layer "B.Cu") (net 3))
 (segment (start 153.4 73.243) (end 142.407 73.243) (width 0.25) (layer "B.Cu") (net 31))
 (segment (start 142.407 73.243) (end 120.27 95.38) (width 0.25) (layer "B.Cu") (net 31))
 (segment (start 143.822489 74.367511) (end 122.81 95.38) (width 0.25) (layer "B.Cu") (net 10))
 (segment (start 177.275489 74.367511) (end 143.822489 74.367511) (width 0.25) (layer "B.Cu") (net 10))
 (segment (start 178.4 73.243) (end 177.275489 74.367511) (width 0.25) (layer "B.Cu") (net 10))
 (segment (start 108.84 103) (end 112.65 103) (width 0.25) (layer "F.Cu") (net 38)))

